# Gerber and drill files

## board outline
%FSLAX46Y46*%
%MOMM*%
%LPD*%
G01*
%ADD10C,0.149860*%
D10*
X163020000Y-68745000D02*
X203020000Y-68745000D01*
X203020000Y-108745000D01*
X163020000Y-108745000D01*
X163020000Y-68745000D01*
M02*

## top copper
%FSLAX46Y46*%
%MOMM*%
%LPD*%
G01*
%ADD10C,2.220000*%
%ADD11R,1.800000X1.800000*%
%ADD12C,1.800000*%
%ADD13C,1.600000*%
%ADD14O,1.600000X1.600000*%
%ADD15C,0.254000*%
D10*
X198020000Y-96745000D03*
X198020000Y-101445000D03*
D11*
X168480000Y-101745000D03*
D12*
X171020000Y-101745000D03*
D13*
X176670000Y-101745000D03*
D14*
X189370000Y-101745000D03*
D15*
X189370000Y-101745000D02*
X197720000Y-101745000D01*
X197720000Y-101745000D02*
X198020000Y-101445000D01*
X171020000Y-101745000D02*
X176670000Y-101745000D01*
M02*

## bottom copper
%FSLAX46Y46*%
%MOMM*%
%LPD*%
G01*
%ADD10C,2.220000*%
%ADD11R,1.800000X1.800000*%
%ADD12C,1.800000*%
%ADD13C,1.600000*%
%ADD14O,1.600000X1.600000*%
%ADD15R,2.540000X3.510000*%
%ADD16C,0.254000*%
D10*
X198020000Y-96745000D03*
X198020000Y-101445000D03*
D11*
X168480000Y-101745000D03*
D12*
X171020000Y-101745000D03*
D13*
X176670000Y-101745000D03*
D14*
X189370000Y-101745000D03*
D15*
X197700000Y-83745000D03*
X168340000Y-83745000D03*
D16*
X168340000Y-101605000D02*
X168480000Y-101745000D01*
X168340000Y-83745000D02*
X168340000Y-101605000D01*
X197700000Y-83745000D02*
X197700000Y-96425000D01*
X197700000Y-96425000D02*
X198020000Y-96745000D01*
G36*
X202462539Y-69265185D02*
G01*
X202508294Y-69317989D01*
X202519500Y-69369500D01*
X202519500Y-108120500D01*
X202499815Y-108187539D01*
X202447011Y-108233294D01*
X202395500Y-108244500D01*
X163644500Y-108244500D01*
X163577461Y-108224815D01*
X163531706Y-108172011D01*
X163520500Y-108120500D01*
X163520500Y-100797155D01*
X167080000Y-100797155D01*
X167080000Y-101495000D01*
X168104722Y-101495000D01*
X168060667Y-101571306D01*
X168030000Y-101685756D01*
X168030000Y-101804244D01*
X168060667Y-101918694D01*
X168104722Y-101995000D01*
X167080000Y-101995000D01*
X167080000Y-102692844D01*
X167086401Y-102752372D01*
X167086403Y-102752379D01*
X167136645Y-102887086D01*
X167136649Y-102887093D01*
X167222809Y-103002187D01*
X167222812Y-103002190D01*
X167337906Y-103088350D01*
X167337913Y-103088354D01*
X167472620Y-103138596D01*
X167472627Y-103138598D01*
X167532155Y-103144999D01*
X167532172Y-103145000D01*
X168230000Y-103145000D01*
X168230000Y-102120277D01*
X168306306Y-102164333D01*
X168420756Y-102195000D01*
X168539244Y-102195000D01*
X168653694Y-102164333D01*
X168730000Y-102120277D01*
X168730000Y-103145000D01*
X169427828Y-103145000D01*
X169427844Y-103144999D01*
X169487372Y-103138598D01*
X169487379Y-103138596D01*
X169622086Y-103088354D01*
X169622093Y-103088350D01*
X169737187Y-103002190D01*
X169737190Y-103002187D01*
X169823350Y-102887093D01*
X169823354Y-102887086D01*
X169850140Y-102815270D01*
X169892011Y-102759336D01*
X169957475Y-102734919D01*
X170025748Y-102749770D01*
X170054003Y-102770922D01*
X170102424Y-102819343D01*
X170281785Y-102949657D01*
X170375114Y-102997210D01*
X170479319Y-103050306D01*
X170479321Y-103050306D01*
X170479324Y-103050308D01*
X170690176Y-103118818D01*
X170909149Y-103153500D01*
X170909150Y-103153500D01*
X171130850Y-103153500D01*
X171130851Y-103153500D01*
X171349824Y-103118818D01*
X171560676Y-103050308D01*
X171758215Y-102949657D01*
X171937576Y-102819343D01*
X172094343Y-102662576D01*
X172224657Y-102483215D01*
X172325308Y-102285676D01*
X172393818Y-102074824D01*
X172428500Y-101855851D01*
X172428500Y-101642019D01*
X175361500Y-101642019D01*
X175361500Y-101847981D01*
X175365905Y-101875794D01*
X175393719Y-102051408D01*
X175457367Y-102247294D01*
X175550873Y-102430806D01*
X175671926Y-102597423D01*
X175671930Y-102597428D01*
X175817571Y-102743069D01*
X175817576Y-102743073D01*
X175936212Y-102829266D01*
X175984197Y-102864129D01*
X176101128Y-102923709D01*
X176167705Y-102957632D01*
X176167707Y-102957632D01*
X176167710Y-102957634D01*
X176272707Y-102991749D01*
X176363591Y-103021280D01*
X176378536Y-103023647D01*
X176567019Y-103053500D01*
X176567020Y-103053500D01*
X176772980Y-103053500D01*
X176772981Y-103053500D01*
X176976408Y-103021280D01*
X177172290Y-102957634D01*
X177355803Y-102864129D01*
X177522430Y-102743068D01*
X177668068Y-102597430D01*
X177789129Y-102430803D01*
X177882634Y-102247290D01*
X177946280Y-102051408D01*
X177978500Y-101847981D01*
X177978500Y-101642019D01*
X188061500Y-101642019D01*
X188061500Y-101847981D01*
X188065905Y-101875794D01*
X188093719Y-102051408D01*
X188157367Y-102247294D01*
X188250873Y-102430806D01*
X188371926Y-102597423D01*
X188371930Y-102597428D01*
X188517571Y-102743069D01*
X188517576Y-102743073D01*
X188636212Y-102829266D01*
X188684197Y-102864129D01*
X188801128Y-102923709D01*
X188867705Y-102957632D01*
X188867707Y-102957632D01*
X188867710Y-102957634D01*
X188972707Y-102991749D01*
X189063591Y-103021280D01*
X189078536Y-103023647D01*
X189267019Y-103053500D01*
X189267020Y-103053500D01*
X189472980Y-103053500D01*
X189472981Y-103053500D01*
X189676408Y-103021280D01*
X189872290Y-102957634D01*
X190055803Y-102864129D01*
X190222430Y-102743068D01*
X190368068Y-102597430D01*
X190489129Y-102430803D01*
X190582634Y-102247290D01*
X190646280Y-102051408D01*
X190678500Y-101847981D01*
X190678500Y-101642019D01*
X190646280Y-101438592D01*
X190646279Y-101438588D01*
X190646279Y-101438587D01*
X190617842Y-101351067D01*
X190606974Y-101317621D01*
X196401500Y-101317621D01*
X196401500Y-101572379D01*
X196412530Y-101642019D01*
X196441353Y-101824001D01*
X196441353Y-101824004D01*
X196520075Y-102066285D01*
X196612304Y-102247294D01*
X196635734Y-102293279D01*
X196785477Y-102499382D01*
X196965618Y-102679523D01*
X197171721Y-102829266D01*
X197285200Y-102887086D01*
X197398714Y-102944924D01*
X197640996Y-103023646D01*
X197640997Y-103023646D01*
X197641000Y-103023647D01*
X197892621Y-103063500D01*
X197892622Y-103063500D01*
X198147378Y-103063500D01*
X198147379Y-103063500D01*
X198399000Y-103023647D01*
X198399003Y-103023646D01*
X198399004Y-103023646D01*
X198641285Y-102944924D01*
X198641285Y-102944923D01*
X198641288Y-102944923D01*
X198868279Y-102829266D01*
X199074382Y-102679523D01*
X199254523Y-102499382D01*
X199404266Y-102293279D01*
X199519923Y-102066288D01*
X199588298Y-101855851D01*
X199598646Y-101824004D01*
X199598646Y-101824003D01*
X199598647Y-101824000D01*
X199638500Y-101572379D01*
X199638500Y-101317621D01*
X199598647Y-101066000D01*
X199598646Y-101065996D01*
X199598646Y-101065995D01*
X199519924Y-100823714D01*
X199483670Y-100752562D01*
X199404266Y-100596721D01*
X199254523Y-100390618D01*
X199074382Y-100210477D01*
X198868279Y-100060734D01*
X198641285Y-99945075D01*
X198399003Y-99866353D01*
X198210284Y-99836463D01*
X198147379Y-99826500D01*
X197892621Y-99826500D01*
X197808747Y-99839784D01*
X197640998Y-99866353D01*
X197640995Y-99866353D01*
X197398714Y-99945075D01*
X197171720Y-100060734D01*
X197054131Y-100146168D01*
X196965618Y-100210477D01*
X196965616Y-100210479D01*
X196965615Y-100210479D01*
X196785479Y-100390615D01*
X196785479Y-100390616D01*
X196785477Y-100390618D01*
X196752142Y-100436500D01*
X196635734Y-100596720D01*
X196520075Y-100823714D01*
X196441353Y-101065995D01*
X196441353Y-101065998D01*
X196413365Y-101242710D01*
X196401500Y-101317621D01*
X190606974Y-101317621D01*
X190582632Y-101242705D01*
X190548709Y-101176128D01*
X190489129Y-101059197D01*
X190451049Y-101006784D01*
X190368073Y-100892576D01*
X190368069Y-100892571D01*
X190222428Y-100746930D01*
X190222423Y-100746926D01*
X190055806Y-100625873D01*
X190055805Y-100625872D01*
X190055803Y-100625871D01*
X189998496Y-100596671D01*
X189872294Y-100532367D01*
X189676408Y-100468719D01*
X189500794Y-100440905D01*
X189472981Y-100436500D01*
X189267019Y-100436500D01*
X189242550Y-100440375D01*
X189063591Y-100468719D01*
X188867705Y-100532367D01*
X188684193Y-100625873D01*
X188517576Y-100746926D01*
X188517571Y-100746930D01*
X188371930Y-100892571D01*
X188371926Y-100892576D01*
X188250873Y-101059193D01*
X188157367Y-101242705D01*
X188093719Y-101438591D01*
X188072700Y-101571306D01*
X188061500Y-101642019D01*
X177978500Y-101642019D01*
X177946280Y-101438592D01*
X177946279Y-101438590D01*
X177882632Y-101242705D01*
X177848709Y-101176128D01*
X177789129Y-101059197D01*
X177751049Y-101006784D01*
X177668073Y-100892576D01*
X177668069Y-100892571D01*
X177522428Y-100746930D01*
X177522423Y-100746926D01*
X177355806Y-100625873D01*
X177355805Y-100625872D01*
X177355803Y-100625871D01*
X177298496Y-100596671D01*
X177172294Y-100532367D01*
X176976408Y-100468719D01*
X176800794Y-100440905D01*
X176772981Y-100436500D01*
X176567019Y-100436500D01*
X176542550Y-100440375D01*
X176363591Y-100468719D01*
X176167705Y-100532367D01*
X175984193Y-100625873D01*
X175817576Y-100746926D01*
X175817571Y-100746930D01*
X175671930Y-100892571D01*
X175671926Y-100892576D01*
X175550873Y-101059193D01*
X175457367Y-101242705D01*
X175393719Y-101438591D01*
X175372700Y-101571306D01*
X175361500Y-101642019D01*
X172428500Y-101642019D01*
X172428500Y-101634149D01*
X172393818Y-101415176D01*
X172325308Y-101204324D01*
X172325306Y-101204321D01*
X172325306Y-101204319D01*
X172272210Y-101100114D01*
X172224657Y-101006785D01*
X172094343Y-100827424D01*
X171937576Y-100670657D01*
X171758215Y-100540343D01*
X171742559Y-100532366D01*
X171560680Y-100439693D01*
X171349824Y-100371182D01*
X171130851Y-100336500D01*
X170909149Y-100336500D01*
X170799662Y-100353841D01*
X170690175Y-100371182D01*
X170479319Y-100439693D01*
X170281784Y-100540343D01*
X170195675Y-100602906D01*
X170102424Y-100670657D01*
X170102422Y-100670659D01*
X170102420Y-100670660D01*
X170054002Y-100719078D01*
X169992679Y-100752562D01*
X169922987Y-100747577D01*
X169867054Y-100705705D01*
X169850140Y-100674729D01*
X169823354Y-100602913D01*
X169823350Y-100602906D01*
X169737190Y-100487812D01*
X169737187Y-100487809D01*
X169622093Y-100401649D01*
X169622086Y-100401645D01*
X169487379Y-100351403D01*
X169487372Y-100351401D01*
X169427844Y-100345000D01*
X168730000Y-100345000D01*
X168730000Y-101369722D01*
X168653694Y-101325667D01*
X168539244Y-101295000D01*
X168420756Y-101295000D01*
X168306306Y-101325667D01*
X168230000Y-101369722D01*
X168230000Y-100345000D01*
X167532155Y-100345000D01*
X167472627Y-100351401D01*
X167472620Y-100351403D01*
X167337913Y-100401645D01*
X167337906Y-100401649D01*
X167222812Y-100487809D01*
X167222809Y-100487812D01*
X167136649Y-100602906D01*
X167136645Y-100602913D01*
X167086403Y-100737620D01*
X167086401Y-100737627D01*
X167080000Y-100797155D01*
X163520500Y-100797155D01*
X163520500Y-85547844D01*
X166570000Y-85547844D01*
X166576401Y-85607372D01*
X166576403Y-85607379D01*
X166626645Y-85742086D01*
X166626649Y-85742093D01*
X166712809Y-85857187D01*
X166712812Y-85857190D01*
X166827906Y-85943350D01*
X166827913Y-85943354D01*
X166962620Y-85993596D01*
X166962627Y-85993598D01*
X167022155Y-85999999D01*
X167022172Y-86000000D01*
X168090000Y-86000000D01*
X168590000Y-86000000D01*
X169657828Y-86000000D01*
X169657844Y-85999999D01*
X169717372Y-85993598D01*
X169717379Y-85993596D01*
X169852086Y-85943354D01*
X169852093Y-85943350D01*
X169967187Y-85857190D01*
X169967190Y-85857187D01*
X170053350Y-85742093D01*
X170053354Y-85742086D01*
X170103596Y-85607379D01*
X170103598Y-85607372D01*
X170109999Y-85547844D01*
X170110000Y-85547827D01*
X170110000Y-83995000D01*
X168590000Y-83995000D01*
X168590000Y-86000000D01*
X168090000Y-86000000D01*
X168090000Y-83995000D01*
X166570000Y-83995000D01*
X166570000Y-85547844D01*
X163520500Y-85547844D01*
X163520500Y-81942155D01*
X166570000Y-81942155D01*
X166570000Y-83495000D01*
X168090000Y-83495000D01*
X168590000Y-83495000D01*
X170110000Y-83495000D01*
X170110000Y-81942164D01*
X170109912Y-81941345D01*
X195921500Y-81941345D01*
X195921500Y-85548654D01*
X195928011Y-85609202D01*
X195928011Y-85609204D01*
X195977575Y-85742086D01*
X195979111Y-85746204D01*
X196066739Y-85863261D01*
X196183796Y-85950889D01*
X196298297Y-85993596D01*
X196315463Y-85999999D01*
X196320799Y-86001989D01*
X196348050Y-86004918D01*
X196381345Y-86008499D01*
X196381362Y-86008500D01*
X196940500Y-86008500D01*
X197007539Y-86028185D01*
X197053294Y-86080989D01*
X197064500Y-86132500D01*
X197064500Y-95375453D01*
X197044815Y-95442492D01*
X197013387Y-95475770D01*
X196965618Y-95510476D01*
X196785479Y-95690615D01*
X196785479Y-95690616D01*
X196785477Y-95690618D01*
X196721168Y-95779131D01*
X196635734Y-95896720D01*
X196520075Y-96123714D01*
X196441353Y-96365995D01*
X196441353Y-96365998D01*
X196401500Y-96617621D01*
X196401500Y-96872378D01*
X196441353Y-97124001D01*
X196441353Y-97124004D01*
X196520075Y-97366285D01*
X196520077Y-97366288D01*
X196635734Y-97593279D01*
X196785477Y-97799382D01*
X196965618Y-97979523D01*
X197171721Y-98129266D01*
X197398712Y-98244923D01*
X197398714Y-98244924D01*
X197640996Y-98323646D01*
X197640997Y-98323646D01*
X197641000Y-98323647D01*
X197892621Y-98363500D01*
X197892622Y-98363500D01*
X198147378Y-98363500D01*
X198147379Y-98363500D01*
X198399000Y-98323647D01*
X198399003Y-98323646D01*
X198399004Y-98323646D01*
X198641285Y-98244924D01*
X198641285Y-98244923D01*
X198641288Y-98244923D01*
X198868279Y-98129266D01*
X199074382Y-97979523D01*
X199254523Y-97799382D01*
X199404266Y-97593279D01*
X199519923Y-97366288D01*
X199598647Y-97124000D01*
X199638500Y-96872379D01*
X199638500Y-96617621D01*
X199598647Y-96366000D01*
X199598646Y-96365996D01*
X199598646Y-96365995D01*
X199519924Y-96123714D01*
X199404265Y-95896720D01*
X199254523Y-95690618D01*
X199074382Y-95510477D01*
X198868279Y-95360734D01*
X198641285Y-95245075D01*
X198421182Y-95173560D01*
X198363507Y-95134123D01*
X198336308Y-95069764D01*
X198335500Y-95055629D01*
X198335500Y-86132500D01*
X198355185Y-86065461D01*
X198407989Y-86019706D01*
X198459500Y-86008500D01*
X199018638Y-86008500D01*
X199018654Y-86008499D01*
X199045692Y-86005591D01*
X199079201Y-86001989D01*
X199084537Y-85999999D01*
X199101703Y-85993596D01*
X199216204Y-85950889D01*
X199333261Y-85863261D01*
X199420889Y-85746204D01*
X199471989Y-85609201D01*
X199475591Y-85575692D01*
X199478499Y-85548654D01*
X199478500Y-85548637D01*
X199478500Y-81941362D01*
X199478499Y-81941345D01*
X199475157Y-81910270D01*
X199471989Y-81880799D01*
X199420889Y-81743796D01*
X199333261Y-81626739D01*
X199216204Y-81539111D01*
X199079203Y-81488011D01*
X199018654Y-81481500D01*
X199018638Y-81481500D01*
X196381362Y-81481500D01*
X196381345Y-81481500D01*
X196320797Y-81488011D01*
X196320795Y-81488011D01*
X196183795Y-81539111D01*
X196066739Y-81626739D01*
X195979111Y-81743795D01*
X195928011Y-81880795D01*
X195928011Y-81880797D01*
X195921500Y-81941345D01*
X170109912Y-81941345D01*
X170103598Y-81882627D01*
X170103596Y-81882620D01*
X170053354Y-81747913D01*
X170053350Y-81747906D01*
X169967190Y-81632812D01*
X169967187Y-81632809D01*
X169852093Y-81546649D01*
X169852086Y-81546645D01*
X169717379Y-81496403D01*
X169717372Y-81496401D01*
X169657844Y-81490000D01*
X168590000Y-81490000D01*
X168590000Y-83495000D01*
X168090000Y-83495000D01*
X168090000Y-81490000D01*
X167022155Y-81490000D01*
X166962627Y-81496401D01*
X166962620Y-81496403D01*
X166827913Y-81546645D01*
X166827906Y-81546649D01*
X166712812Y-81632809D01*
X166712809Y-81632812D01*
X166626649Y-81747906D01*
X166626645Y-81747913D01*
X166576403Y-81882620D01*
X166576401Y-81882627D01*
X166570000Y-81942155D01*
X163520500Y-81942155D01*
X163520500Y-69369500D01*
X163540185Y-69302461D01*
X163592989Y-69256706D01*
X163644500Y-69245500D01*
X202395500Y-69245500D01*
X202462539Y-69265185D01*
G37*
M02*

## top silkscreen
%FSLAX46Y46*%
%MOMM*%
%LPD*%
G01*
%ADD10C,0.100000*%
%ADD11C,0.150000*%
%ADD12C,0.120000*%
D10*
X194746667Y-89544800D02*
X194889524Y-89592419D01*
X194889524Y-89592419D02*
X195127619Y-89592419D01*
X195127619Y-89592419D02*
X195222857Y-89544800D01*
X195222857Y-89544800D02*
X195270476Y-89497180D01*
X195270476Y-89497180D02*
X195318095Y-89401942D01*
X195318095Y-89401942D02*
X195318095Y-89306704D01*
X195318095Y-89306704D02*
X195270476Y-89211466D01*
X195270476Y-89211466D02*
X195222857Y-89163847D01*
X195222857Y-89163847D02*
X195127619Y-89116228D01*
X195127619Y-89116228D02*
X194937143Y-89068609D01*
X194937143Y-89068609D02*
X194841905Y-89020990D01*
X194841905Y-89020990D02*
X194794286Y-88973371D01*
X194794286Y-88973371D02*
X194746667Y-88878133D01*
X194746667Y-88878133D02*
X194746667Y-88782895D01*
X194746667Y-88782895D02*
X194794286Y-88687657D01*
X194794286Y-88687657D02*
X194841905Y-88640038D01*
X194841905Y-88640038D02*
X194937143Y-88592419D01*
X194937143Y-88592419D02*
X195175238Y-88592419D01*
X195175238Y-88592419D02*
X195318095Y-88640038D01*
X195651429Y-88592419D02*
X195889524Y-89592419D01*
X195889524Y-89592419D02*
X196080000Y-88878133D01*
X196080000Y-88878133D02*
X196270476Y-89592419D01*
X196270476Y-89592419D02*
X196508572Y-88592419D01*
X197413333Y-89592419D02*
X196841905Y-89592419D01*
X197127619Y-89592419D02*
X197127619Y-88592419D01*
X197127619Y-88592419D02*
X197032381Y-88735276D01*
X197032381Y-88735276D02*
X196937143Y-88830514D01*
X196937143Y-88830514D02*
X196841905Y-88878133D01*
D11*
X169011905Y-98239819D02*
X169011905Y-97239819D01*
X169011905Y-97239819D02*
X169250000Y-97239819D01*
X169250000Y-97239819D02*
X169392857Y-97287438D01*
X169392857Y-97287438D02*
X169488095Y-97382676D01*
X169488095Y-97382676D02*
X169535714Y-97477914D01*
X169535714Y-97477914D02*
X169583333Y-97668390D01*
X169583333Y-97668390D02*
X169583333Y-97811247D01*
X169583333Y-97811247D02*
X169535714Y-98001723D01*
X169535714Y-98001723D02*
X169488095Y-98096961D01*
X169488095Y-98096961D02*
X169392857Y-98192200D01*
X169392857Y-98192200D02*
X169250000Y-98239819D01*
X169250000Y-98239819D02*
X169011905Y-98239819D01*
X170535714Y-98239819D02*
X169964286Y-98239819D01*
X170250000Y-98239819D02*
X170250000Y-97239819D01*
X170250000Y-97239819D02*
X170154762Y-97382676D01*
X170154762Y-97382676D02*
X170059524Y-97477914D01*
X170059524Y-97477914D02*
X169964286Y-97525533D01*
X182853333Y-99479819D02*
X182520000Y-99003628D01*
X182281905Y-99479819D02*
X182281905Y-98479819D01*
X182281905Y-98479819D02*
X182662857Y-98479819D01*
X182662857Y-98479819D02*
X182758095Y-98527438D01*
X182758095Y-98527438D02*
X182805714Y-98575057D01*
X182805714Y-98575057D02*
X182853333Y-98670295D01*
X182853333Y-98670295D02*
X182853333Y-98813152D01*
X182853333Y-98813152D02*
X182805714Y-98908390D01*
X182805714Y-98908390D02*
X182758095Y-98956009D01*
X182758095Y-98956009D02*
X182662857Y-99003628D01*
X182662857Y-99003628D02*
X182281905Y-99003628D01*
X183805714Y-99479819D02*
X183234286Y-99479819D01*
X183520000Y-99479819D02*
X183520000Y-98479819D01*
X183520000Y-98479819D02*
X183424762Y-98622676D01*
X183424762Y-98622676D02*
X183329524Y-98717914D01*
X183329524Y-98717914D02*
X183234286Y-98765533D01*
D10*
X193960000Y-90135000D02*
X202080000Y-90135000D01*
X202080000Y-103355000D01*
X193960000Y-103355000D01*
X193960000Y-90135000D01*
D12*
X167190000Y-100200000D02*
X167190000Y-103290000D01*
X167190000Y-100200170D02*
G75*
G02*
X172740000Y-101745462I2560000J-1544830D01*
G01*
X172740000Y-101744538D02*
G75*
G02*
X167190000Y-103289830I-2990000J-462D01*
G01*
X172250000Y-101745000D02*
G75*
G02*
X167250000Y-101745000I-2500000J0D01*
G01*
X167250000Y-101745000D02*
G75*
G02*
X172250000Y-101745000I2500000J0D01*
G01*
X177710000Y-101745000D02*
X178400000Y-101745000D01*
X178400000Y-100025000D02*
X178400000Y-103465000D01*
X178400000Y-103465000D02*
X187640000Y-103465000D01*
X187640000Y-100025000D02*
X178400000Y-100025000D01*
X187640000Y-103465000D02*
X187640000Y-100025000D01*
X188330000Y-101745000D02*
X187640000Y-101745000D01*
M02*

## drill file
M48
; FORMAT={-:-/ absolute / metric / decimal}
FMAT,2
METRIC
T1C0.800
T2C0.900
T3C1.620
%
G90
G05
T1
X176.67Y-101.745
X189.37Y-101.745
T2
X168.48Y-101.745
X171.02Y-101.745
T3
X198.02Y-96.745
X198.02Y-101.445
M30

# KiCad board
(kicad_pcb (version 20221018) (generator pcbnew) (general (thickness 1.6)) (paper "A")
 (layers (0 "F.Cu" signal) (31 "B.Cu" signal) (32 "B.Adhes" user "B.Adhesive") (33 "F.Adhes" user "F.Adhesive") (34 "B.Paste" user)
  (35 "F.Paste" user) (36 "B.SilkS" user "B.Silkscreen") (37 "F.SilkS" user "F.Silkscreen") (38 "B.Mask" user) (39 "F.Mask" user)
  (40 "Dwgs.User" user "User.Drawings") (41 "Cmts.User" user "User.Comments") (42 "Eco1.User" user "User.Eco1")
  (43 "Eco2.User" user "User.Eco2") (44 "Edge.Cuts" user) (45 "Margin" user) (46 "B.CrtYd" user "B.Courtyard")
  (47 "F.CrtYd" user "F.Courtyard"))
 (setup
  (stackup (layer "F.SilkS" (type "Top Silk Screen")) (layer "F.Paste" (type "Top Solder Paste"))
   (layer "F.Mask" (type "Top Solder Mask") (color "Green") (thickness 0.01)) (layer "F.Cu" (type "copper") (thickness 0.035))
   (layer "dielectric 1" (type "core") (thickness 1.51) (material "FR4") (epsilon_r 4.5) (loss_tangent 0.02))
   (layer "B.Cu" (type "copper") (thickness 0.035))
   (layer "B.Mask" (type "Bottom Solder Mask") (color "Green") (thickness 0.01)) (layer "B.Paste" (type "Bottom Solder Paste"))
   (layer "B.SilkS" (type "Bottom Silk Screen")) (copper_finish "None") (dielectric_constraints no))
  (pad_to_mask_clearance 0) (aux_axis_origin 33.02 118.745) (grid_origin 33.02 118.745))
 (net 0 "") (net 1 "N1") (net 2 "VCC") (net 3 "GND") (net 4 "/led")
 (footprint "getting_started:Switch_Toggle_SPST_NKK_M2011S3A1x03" (layer "F.Cu") (at 198.02 92.045)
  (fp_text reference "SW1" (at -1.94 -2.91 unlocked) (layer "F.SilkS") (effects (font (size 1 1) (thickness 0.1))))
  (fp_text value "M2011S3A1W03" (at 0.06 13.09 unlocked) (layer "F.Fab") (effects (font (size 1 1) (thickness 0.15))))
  (fp_rect (start 4.06 -1.91) (end -4.06 11.31) (stroke (width 0.1) (type default)) (fill none) (layer "F.SilkS"))
  (pad "2" thru_hole circle (at 0 4.7) (size 2.22 2.22) (drill 1.62) (layers "*.Cu" "*.Mask") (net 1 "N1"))
  (pad "3" thru_hole circle (at 0 9.4) (size 2.22 2.22) (drill 1.62) (layers "*.Cu" "*.Mask") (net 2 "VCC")))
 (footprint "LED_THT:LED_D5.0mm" (layer "F.Cu") (at 168.48 101.745)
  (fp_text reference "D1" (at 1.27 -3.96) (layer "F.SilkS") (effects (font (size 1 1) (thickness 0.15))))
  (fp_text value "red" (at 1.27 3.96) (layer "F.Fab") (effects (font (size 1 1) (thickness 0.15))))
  (fp_line (start -1.29 -1.545) (end -1.29 1.545) (stroke (width 0.12) (type solid)) (layer "F.SilkS"))
  (fp_arc (start -1.29 -1.54483) (mid 2.072002 -2.880433) (end 4.26 0.000462) (stroke (width 0.12) (type solid)) (layer "F.SilkS"))
  (fp_arc (start 4.26 -0.000462) (mid 2.072002 2.880433) (end -1.29 1.54483) (stroke (width 0.12) (type solid)) (layer "F.SilkS"))
  (fp_circle (center 1.27 0) (end 3.77 0) (stroke (width 0.12) (type solid)) (fill none) (layer "F.SilkS"))
  (pad "1" thru_hole rect (at 0 0) (size 1.8 1.8) (drill 0.9) (layers "*.Cu" "*.Mask") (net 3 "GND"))
  (pad "2" thru_hole circle (at 2.54 0) (size 1.8 1.8) (drill 0.9) (layers "*.Cu" "*.Mask") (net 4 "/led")))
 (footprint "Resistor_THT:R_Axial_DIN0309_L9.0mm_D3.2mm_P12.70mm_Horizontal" (layer "F.Cu") (at 176.67 101.745)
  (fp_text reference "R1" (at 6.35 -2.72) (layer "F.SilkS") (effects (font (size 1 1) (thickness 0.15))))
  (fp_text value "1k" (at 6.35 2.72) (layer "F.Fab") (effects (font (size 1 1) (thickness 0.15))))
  (fp_line (start 1.04 0) (end 1.73 0) (stroke (width 0.12) (type solid)) (layer "F.SilkS"))
  (fp_line (start 1.73 -1.72) (end 1.73 1.72) (stroke (width 0.12) (type solid)) (layer "F.SilkS"))
  (fp_line (start 1.73 1.72) (end 10.97 1.72) (stroke (width 0.12) (type solid)) (layer "F.SilkS"))
  (fp_line (start 10.97 -1.72) (end 1.73 -1.72) (stroke (width 0.12) (type solid)) (layer "F.SilkS"))
  (fp_line (start 10.97 1.72) (end 10.97 -1.72) (stroke (width 0.12) (type solid)) (layer "F.SilkS"))
  (fp_line (start 11.66 0) (end 10.97 0) (stroke (width 0.12) (type solid)) (layer "F.SilkS"))
  (pad "1" thru_hole circle (at 0 0) (size 1.6 1.6) (drill 0.8) (layers "*.Cu" "*.Mask") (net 4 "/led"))
  (pad "2" thru_hole oval (at 12.7 0) (size 1.6 1.6) (drill 0.8) (layers "*.Cu" "*.Mask") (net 2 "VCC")))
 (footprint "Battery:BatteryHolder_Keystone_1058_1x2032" (layer "B.Cu") (at 183.02 83.745 180)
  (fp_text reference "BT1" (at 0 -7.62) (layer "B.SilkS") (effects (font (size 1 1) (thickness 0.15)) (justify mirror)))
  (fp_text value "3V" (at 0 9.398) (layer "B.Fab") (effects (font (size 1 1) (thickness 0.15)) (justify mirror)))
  (pad "1" smd rect (at -14.68 0 180) (size 2.54 3.51) (layers "B.Cu" "B.Paste" "B.Mask") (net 1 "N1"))
  (pad "2" smd rect (at 14.68 0 180) (size 2.54 3.51) (layers "B.Cu" "B.Paste" "B.Mask") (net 3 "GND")))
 (gr_rect (start 163.02 68.745) (end 203.02 108.745) (stroke (width 0.14986) (type default)) (fill none) (layer "Edge.Cuts"))
 (segment (start 168.34 101.605) (end 168.48 101.745) (width 0.254) (layer "B.Cu") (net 3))
 (segment (start 168.34 83.745) (end 168.34 101.605) (width 0.254) (layer "B.Cu") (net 3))
 (segment (start 189.37 101.745) (end 197.72 101.745) (width 0.254) (layer "F.Cu") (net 2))
 (segment (start 197.72 101.745) (end 198.02 101.445) (width 0.254) (layer "F.Cu") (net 2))
 (segment (start 171.02 101.745) (end 176.67 101.745) (width 0.254) (layer "F.Cu") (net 4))
 (segment (start 197.7 83.745) (end 197.7 96.425) (width 0.254) (layer "B.Cu") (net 1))
 (segment (start 197.7 96.425) (end 198.02 96.745) (width 0.254) (layer "B.Cu") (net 1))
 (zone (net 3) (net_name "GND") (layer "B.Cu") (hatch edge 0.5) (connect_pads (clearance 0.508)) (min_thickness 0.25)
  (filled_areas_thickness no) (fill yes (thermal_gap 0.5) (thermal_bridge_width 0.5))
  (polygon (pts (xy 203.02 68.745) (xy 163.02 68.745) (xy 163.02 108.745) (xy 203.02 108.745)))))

